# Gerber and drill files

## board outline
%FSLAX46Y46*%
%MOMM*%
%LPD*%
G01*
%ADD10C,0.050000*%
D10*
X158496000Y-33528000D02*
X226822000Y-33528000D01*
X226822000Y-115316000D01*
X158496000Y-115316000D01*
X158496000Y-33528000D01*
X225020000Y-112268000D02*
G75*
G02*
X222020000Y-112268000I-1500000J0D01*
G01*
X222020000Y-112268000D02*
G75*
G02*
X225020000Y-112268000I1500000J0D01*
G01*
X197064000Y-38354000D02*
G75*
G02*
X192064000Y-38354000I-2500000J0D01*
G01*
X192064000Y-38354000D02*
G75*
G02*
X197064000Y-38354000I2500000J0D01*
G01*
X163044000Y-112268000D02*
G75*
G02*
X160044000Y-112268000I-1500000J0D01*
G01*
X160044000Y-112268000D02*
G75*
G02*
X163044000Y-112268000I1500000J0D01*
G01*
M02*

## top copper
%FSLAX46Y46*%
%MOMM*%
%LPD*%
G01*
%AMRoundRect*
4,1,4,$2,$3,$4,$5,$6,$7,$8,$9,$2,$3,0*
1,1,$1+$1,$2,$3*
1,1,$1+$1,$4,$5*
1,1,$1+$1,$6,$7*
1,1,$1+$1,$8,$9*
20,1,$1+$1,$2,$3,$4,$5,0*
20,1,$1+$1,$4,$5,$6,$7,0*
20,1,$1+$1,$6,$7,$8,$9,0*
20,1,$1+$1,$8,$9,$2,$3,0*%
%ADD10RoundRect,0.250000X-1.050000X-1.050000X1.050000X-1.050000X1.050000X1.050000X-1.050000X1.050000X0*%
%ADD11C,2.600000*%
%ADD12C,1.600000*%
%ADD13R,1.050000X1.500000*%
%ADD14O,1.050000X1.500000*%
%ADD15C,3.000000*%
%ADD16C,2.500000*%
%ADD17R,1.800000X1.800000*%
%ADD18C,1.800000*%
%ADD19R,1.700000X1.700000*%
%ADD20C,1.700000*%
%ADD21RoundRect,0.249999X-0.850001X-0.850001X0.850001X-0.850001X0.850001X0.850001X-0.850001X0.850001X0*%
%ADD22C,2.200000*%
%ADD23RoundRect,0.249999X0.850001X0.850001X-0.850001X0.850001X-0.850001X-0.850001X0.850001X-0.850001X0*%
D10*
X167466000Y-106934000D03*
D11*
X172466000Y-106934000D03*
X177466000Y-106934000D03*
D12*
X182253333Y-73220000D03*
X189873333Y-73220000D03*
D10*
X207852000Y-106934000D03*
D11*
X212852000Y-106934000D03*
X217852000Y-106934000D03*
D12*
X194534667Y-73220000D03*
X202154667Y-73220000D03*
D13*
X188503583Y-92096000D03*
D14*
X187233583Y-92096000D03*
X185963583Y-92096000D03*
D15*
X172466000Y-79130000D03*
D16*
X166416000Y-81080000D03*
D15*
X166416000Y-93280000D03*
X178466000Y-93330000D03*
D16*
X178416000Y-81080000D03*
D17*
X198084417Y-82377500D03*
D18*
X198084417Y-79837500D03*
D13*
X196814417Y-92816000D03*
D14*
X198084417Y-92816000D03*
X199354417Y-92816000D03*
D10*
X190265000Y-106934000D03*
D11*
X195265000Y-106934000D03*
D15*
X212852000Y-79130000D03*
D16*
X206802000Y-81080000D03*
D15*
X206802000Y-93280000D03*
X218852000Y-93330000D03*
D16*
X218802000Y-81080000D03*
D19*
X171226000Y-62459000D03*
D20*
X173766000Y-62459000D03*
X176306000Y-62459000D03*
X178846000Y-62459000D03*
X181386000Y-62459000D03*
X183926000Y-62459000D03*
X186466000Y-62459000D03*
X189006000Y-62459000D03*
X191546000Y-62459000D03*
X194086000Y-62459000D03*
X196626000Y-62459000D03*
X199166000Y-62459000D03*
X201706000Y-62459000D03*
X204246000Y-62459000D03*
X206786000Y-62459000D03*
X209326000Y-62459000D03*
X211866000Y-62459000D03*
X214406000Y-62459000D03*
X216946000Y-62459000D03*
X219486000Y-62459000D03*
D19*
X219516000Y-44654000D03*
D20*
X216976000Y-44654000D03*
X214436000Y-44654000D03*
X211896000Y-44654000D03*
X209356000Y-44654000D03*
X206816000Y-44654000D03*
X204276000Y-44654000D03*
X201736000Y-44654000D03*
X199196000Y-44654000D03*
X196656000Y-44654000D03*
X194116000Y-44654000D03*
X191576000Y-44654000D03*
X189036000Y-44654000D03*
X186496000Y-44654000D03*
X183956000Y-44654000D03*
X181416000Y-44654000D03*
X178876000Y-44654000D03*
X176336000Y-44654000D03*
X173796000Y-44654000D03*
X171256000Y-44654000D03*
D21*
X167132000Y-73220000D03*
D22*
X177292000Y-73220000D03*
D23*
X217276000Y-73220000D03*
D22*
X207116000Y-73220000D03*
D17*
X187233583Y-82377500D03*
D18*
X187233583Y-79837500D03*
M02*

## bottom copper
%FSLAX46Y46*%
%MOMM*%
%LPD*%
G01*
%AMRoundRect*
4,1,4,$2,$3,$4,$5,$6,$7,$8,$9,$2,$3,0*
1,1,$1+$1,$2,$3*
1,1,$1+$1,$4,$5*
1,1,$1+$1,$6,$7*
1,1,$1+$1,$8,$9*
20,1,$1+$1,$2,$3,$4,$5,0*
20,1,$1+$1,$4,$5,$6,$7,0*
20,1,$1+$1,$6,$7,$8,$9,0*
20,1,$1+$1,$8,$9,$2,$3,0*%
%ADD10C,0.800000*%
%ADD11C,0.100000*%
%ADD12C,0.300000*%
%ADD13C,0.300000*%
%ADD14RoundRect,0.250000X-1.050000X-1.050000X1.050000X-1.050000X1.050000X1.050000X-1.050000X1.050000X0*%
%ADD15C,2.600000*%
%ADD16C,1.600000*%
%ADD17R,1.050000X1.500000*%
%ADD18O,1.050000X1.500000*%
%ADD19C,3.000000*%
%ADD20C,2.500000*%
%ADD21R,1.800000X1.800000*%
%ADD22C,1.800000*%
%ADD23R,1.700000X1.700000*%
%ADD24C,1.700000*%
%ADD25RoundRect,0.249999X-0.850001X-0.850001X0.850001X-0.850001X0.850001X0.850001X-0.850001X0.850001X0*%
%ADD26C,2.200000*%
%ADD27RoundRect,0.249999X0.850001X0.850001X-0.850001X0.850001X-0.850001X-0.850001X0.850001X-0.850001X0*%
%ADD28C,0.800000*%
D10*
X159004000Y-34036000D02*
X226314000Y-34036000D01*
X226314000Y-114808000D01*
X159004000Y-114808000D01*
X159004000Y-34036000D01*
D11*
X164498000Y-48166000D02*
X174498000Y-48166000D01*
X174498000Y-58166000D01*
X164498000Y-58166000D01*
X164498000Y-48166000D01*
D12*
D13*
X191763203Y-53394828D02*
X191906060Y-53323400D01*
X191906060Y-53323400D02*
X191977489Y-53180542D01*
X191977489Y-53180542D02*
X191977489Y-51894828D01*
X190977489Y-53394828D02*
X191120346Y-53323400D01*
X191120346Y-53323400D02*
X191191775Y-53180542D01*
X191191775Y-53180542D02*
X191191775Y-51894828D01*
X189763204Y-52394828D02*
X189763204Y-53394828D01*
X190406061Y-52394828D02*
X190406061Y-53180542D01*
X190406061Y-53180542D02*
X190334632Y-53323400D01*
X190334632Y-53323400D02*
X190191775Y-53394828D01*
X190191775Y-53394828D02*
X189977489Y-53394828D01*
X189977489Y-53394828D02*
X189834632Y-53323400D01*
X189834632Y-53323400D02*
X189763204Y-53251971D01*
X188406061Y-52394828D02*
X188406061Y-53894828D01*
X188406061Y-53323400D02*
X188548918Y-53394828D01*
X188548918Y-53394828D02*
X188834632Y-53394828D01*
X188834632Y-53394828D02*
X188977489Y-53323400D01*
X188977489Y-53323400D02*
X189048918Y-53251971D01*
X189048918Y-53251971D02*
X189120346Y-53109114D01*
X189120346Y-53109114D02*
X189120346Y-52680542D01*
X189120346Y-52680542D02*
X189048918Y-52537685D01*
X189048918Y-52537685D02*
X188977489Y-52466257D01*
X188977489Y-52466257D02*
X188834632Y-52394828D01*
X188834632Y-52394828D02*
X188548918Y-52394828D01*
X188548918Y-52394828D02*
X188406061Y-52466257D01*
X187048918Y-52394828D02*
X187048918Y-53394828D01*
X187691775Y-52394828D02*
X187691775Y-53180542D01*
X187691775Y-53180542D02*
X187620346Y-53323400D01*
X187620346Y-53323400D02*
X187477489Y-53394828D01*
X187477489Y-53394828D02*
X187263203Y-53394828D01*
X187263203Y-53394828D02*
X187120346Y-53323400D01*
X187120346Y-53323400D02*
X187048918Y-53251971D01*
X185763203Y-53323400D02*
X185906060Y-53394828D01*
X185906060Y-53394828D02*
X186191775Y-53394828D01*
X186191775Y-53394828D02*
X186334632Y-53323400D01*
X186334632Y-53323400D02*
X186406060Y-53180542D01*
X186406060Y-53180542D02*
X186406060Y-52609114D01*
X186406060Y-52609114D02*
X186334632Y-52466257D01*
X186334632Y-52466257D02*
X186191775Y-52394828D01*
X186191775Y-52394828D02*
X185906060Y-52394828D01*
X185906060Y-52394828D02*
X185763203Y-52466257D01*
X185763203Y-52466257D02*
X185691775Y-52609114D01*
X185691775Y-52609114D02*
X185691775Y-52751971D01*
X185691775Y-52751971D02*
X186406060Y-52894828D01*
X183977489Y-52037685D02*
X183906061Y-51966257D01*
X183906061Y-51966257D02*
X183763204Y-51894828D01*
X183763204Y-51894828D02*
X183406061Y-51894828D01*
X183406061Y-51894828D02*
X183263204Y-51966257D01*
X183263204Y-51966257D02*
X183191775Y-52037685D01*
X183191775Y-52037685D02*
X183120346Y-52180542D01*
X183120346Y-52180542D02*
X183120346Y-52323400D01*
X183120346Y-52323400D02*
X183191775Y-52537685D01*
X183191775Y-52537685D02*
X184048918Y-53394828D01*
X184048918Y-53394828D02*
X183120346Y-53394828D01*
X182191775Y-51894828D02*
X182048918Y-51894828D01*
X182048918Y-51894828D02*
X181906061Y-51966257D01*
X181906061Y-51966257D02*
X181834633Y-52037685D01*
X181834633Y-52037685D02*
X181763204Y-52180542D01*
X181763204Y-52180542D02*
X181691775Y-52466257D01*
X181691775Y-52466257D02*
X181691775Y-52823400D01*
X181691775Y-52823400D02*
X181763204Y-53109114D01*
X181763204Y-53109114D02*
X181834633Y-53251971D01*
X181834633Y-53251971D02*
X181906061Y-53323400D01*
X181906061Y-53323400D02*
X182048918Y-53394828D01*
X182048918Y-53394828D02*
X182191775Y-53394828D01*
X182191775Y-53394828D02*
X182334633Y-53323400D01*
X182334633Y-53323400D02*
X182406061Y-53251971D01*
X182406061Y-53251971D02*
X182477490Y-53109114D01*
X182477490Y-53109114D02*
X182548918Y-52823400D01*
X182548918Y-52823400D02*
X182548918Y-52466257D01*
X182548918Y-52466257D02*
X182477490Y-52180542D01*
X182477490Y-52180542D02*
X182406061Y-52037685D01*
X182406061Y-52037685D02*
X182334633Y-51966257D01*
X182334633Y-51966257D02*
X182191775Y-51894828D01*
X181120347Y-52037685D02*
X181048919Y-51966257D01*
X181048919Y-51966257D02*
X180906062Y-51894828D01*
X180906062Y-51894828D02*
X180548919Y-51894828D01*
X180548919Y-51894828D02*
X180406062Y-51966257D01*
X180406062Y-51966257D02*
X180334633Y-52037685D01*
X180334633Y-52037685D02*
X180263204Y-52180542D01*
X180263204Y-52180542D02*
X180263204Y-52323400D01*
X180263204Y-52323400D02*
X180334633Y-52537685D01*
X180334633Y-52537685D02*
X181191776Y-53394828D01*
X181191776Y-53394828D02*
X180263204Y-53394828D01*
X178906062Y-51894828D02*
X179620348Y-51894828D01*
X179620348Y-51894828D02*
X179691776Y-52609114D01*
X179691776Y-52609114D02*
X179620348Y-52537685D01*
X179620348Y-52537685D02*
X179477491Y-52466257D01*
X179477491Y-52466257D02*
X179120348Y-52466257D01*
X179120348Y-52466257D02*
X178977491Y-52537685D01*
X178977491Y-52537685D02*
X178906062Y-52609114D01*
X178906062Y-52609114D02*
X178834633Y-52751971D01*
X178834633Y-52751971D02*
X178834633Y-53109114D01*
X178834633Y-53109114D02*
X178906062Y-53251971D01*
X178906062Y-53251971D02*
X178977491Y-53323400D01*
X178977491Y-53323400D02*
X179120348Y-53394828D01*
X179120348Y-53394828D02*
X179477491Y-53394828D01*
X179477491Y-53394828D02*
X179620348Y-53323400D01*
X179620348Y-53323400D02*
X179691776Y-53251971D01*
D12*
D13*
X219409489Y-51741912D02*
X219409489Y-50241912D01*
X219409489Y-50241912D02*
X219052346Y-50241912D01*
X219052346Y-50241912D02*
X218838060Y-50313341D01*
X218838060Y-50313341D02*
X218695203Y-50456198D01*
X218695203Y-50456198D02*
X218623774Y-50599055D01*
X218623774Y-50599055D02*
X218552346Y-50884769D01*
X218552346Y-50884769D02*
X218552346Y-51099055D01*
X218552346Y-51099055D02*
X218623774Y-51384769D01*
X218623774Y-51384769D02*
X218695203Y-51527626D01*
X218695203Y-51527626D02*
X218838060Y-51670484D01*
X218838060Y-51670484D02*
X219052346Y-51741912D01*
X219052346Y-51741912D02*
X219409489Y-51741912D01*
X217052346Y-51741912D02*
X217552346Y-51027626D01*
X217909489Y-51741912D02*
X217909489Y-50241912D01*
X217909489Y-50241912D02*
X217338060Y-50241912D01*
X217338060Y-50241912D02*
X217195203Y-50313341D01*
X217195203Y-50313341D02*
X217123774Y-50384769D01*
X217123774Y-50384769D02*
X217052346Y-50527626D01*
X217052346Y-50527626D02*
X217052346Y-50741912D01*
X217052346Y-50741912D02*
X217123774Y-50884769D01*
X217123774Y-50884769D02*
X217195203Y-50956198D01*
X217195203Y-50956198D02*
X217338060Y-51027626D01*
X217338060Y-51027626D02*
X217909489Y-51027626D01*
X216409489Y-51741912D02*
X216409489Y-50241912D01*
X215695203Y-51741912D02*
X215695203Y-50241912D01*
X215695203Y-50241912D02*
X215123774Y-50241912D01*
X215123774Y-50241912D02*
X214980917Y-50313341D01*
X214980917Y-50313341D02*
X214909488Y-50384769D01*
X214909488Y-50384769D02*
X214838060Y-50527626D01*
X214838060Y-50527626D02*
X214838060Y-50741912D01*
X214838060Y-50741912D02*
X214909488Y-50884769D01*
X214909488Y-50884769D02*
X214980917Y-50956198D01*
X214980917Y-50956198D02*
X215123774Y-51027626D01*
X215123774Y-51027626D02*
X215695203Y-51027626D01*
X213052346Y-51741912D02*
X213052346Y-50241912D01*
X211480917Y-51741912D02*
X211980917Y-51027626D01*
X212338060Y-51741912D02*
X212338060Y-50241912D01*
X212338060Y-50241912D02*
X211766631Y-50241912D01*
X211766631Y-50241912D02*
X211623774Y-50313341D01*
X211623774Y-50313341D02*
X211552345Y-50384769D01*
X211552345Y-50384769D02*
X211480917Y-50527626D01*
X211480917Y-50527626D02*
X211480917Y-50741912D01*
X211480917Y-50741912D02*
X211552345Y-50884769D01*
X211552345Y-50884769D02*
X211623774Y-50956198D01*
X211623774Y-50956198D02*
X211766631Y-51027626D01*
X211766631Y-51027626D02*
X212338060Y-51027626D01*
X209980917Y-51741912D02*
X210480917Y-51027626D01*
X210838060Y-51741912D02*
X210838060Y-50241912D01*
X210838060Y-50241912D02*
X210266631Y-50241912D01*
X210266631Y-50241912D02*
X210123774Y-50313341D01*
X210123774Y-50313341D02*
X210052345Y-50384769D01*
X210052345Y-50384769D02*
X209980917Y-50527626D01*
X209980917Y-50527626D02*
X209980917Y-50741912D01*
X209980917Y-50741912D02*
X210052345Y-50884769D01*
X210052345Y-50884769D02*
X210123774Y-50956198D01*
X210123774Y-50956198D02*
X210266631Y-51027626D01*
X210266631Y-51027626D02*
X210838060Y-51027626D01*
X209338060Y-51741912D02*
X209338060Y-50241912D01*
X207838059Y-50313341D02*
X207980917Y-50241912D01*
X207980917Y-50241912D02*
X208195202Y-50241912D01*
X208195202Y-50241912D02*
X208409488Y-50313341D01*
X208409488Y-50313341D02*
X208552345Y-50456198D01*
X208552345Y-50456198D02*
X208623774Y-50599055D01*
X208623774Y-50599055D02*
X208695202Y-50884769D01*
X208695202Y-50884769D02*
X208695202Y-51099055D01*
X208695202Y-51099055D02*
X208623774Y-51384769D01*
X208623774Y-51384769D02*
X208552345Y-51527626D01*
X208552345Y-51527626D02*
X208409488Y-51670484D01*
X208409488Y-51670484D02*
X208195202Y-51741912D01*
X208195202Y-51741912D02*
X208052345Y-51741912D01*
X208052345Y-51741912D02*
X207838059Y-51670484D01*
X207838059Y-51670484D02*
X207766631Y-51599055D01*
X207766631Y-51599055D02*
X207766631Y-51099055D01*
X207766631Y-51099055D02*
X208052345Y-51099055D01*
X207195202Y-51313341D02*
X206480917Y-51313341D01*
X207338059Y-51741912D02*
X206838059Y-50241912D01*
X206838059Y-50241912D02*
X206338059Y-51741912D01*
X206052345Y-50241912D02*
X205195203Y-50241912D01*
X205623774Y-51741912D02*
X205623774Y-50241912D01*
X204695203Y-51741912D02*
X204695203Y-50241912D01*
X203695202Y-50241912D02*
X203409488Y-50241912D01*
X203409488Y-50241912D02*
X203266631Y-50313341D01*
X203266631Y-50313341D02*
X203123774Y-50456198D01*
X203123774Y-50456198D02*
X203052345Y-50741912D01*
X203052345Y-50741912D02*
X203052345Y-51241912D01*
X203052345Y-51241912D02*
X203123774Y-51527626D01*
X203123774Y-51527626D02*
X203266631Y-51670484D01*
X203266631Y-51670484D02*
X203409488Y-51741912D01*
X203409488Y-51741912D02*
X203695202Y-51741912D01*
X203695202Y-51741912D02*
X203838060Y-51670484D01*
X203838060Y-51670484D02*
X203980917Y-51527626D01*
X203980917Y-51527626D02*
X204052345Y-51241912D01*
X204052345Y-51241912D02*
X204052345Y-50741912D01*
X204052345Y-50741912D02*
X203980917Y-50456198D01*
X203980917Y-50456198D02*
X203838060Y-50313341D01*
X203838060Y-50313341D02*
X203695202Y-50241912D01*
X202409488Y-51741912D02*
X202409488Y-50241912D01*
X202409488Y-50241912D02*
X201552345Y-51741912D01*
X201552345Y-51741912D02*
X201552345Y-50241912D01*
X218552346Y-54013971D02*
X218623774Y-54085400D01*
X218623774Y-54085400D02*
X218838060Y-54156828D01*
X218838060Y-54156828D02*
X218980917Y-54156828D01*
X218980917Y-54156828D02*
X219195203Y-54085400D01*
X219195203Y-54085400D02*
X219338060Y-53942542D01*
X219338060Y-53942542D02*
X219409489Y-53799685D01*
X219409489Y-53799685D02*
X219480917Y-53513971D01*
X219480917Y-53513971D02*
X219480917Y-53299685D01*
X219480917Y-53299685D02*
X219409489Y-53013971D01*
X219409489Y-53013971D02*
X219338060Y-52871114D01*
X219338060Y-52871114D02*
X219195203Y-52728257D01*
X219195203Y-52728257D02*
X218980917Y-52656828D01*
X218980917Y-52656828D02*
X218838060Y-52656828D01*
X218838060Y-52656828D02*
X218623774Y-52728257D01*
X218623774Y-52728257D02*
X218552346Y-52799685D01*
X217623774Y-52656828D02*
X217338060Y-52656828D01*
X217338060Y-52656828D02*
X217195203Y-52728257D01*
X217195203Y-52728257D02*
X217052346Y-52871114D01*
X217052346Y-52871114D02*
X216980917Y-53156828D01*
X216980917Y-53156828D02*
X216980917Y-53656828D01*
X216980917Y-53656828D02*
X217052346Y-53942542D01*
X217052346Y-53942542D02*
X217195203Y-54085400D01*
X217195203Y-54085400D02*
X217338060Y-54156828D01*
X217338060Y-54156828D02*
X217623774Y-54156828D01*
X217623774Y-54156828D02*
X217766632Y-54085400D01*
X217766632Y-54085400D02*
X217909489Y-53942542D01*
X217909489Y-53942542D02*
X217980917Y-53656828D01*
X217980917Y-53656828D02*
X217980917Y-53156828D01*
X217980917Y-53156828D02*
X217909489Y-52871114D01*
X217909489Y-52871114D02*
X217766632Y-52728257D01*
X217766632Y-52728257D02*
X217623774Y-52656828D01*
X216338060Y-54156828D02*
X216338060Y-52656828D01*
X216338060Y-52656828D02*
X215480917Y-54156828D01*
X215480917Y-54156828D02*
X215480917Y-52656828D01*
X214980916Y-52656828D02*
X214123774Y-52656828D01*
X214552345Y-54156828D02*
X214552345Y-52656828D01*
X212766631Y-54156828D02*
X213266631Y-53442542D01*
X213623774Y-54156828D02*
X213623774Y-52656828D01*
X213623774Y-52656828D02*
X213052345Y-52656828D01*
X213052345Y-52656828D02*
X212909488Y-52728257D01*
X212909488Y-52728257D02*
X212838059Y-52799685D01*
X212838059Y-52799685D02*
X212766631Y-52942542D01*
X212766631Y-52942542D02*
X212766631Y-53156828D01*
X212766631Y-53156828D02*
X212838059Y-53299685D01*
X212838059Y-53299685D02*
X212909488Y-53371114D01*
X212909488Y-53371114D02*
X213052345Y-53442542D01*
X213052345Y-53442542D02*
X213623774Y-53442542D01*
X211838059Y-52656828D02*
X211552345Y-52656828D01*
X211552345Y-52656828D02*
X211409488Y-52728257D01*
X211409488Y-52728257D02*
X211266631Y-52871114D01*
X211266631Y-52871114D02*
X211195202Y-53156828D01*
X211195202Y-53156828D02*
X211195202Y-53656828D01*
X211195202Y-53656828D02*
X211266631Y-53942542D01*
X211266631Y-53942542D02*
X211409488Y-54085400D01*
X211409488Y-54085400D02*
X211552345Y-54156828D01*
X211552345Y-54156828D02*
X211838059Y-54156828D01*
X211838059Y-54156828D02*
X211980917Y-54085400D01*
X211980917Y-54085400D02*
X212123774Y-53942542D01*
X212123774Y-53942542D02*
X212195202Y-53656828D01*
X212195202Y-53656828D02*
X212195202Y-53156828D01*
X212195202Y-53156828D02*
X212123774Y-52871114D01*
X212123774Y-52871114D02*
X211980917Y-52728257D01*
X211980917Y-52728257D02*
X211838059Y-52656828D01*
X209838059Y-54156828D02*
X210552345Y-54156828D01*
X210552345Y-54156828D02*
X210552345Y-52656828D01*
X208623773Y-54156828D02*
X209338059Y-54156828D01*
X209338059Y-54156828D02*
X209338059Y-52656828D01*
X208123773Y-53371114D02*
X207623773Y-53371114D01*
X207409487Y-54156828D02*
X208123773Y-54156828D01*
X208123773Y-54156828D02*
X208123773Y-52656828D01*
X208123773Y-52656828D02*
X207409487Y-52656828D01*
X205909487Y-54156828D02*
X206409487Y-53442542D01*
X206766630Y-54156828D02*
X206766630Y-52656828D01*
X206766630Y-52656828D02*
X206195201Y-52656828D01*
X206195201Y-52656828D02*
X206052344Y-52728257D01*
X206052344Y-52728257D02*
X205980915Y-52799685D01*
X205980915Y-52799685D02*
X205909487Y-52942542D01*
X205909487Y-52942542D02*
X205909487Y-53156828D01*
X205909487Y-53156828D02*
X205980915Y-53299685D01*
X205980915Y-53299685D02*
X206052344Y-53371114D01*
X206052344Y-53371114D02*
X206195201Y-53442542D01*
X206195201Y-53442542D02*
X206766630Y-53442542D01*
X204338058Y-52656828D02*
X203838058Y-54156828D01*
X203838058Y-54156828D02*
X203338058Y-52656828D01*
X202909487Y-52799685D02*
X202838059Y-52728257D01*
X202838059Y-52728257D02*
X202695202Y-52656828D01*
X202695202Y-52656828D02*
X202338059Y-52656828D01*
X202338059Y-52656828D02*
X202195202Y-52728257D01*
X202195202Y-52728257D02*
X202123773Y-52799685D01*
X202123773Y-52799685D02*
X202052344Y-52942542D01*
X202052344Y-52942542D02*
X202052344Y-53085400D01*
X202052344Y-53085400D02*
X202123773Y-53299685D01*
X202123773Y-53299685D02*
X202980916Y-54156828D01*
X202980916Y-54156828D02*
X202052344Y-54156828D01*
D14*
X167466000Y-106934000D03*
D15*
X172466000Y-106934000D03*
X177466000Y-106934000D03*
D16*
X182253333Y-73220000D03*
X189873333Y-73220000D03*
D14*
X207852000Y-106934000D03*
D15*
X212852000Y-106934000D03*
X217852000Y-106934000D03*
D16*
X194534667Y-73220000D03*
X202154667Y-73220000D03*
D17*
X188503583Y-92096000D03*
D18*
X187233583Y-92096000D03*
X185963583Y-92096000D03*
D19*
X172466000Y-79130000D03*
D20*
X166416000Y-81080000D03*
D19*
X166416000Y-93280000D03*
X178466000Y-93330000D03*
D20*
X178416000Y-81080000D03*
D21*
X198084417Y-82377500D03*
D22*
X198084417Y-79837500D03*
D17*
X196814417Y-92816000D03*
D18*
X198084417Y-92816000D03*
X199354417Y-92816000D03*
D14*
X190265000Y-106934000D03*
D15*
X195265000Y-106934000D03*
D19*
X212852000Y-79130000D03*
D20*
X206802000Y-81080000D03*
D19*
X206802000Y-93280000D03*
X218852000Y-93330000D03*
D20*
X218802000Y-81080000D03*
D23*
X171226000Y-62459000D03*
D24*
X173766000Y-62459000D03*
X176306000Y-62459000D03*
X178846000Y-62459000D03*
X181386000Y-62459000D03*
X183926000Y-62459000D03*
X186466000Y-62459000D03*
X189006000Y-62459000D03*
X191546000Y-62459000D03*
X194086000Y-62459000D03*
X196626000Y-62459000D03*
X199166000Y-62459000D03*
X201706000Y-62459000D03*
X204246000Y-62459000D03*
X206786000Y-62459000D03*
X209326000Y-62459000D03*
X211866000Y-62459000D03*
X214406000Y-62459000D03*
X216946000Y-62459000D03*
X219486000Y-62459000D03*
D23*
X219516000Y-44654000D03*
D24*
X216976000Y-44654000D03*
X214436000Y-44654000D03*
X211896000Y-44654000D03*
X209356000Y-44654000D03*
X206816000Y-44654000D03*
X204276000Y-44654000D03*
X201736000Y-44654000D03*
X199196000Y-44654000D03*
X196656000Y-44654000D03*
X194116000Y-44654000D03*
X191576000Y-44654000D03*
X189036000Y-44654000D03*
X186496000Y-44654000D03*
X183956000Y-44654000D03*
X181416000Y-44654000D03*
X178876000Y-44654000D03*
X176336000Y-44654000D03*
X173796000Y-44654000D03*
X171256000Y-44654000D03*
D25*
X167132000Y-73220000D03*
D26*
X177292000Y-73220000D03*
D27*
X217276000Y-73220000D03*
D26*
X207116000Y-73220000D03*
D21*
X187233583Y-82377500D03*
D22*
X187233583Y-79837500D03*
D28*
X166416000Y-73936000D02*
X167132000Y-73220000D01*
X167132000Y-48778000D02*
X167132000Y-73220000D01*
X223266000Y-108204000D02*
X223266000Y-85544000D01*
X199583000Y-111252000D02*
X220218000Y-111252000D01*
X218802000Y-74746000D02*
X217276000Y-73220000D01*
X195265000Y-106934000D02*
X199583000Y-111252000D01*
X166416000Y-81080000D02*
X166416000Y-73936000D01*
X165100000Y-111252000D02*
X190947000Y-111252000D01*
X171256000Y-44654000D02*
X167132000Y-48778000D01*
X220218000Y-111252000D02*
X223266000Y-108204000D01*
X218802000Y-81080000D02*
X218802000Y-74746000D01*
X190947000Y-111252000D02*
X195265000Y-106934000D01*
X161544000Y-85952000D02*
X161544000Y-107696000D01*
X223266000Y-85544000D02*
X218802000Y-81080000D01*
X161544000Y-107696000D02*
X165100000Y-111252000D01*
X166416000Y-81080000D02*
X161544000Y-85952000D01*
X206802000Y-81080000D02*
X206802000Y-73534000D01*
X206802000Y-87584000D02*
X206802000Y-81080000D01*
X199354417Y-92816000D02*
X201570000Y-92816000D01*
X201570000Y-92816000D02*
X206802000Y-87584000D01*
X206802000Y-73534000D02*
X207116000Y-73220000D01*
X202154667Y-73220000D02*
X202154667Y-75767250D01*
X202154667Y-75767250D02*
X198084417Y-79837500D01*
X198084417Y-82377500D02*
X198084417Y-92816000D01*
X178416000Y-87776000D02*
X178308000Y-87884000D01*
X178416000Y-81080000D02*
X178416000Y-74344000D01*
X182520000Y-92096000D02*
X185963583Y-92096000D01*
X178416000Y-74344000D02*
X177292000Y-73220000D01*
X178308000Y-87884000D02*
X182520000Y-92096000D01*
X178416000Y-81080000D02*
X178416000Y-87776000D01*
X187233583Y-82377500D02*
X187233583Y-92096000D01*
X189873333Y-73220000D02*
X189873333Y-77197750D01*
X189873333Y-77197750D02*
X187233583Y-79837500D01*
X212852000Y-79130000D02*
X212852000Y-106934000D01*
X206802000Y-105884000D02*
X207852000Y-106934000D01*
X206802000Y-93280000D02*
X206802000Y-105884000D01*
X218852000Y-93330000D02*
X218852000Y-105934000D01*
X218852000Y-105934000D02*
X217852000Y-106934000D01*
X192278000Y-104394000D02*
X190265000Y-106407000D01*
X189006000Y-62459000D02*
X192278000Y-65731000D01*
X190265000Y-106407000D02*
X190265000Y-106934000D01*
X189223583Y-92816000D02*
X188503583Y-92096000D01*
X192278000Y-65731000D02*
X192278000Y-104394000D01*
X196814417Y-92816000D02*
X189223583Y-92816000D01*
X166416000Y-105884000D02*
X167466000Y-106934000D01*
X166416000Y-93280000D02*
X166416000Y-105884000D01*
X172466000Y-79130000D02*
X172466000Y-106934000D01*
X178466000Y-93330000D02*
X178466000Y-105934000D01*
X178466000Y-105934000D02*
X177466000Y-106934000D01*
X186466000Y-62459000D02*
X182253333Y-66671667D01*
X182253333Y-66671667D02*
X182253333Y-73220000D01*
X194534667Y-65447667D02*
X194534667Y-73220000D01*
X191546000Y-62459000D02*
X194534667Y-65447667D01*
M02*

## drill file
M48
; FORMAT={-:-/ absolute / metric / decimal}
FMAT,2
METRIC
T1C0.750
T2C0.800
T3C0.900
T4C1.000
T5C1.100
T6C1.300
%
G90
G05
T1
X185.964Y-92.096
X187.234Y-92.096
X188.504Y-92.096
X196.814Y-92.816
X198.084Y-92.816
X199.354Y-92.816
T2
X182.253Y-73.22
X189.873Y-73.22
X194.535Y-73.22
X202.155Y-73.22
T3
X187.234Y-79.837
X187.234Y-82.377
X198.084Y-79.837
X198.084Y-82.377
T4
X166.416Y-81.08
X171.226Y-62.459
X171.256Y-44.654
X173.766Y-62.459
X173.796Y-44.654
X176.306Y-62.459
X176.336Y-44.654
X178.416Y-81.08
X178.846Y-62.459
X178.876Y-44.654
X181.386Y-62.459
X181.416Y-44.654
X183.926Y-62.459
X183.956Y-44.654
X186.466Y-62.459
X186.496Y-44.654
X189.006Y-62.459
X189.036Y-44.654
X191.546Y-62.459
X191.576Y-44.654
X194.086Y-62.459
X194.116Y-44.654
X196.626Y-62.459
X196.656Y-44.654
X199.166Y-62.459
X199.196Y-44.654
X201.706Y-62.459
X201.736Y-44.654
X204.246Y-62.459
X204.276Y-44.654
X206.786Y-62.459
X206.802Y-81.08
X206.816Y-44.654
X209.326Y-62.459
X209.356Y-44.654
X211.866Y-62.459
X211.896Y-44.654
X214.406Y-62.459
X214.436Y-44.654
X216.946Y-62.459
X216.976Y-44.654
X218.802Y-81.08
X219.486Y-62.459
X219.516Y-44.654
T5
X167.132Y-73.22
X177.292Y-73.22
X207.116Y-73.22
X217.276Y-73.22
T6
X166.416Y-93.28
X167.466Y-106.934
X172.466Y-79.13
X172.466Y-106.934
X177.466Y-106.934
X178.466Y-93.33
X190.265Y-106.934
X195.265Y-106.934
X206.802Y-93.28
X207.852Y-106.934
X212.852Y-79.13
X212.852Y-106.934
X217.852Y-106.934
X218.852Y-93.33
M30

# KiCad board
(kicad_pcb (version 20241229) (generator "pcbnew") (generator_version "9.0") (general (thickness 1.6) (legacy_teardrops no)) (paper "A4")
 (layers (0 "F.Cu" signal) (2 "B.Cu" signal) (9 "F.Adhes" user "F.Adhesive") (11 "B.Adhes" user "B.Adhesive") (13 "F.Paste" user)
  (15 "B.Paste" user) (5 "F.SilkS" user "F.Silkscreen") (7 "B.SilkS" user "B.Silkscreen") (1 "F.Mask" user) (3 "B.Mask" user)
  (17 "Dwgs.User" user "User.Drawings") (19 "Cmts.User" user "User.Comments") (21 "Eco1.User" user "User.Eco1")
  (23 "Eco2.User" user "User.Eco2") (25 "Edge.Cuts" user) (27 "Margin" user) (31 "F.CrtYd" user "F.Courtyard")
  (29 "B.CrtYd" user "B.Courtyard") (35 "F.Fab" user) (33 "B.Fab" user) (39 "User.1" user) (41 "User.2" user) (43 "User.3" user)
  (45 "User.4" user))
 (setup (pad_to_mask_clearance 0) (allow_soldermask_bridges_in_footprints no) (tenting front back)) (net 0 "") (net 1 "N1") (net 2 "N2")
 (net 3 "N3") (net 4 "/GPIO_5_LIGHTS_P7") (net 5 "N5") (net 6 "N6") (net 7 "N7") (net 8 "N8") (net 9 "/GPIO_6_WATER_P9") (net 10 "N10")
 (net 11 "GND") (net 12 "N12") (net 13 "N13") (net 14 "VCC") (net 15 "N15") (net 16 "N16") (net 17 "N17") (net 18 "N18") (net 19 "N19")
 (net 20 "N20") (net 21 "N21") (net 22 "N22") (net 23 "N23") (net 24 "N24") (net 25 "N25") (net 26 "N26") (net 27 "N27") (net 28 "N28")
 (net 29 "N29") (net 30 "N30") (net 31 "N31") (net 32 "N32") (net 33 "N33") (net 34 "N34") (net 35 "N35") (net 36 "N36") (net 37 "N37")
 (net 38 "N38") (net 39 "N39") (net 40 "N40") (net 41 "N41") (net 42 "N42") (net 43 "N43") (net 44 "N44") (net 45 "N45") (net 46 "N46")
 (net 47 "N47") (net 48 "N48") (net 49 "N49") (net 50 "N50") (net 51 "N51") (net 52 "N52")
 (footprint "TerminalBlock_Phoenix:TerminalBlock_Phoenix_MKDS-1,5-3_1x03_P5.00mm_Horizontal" (layer "F.Cu") (at 167.466 106.934)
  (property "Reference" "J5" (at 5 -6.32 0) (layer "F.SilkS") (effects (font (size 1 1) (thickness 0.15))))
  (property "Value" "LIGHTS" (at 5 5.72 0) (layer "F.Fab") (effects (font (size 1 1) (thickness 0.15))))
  (pad "1" thru_hole roundrect (at 0 0) (size 2.6 2.6) (drill 1.3) (layers "*.Cu" "*.Mask") (remove_unused_layers no)
   (roundrect_rratio 0.096154) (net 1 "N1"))
  (pad "2" thru_hole circle (at 5 0) (size 2.6 2.6) (drill 1.3) (layers "*.Cu" "*.Mask") (remove_unused_layers no) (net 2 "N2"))
  (pad "3" thru_hole circle (at 10 0) (size 2.6 2.6) (drill 1.3) (layers "*.Cu" "*.Mask") (remove_unused_layers no) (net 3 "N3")))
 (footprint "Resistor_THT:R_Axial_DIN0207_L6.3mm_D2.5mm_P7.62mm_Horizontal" (layer "F.Cu") (at 182.253333 73.22)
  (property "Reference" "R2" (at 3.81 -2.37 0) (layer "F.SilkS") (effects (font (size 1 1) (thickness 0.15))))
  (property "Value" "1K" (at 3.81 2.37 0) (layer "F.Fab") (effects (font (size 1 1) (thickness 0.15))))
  (pad "1" thru_hole circle (at 0 0) (size 1.6 1.6) (drill 0.8) (layers "*.Cu" "*.Mask") (remove_unused_layers no)
   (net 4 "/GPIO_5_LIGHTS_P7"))
  (pad "2" thru_hole circle (at 7.62 0) (size 1.6 1.6) (drill 0.8) (layers "*.Cu" "*.Mask") (remove_unused_layers no) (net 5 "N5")))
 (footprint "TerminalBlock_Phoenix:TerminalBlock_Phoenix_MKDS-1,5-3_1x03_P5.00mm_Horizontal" (layer "F.Cu") (at 207.852 106.934)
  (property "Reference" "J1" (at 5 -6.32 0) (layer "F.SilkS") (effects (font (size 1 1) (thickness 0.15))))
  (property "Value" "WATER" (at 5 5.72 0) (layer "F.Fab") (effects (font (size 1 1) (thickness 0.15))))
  (pad "1" thru_hole roundrect (at 0 0) (size 2.6 2.6) (drill 1.3) (layers "*.Cu" "*.Mask") (remove_unused_layers no)
   (roundrect_rratio 0.096154) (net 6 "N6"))
  (pad "2" thru_hole circle (at 5 0) (size 2.6 2.6) (drill 1.3) (layers "*.Cu" "*.Mask") (remove_unused_layers no) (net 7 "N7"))
  (pad "3" thru_hole circle (at 10 0) (size 2.6 2.6) (drill 1.3) (layers "*.Cu" "*.Mask") (remove_unused_layers no) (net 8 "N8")))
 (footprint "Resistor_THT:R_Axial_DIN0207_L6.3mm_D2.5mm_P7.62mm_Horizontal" (layer "F.Cu") (at 194.534667 73.22)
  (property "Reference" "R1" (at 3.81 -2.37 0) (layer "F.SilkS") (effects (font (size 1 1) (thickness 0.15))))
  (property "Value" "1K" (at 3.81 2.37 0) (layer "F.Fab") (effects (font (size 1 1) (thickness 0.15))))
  (pad "1" thru_hole circle (at 0 0) (size 1.6 1.6) (drill 0.8) (layers "*.Cu" "*.Mask") (remove_unused_layers no)
   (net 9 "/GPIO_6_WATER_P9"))
  (pad "2" thru_hole circle (at 7.62 0) (size 1.6 1.6) (drill 0.8) (layers "*.Cu" "*.Mask") (remove_unused_layers no) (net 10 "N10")))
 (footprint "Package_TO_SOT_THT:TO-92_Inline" (layer "F.Cu") (at 188.503583 92.096 180)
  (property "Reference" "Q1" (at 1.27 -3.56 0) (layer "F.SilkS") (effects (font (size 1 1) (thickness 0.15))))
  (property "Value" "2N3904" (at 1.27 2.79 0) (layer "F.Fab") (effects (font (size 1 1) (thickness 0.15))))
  (pad "1" thru_hole rect (at 0 0 180) (size 1.05 1.5) (drill 0.75) (layers "*.Cu" "*.Mask") (remove_unused_layers no) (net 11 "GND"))
  (pad "2" thru_hole oval (at 1.27 0 180) (size 1.05 1.5) (drill 0.75) (layers "*.Cu" "*.Mask") (remove_unused_layers no) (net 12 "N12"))
  (pad "3" thru_hole oval (at 2.54 0 180) (size 1.05 1.5) (drill 0.75) (layers "*.Cu" "*.Mask") (remove_unused_layers no) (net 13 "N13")))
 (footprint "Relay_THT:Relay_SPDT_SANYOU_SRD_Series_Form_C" (layer "F.Cu") (at 172.466 79.13 -90)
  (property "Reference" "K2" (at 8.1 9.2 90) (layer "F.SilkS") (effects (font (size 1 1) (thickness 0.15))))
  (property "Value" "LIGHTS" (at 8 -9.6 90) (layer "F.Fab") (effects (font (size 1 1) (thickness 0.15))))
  (pad "1" thru_hole circle (at 0 0) (size 3 3) (drill 1.3) (layers "*.Cu" "*.Mask") (remove_unused_layers no) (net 2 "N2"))
  (pad "2" thru_hole circle (at 1.95 6.05) (size 2.5 2.5) (drill 1) (layers "*.Cu" "*.Mask") (remove_unused_layers no) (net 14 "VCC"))
  (pad "3" thru_hole circle (at 14.15 6.05) (size 3 3) (drill 1.3) (layers "*.Cu" "*.Mask") (remove_unused_layers no) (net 1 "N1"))
  (pad "4" thru_hole circle (at 14.2 -6) (size 3 3) (drill 1.3) (layers "*.Cu" "*.Mask") (remove_unused_layers no) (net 3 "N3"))
  (pad "5" thru_hole circle (at 1.95 -5.95) (size 2.5 2.5) (drill 1) (layers "*.Cu" "*.Mask") (remove_unused_layers no) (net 13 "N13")))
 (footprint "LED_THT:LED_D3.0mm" (layer "F.Cu") (at 198.084417 82.3775 90)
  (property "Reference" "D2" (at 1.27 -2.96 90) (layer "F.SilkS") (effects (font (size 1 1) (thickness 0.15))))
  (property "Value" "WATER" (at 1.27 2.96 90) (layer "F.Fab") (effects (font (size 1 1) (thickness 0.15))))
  (pad "1" thru_hole rect (at 0 0 90) (size 1.8 1.8) (drill 0.9) (layers "*.Cu" "*.Mask") (remove_unused_layers no) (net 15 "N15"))
  (pad "2" thru_hole circle (at 2.54 0 90) (size 1.8 1.8) (drill 0.9) (layers "*.Cu" "*.Mask") (remove_unused_layers no) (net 10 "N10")))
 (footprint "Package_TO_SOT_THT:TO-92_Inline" (layer "F.Cu") (at 196.814417 92.816)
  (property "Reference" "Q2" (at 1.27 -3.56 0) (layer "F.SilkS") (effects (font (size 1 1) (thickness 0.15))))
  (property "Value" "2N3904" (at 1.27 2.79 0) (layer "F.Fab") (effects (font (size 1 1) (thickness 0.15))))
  (pad "1" thru_hole rect (at 0 0) (size 1.05 1.5) (drill 0.75) (layers "*.Cu" "*.Mask") (remove_unused_layers no) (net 11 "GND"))
  (pad "2" thru_hole oval (at 1.27 0) (size 1.05 1.5) (drill 0.75) (layers "*.Cu" "*.Mask") (remove_unused_layers no) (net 15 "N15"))
  (pad "3" thru_hole oval (at 2.54 0) (size 1.05 1.5) (drill 0.75) (layers "*.Cu" "*.Mask") (remove_unused_layers no) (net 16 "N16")))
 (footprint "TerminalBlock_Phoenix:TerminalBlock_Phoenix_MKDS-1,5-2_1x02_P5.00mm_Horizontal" (layer "F.Cu") (at 190.265 106.934)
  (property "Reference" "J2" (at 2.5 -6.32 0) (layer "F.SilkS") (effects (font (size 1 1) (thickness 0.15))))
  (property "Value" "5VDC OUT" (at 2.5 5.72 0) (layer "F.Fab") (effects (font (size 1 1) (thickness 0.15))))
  (pad "1" thru_hole roundrect (at 0 0) (size 2.6 2.6) (drill 1.3) (layers "*.Cu" "*.Mask") (remove_unused_layers no)
   (roundrect_rratio 0.096154) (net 11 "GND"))
  (pad "2" thru_hole circle (at 5 0) (size 2.6 2.6) (drill 1.3) (layers "*.Cu" "*.Mask") (remove_unused_layers no) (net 14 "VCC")))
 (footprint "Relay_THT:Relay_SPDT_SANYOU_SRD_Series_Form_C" (layer "F.Cu") (at 212.852 79.13 -90)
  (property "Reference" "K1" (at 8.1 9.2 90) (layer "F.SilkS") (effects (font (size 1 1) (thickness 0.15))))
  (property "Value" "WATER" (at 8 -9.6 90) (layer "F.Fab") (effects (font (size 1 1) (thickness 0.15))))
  (pad "1" thru_hole circle (at 0 0) (size 3 3) (drill 1.3) (layers "*.Cu" "*.Mask") (remove_unused_layers no) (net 7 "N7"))
  (pad "2" thru_hole circle (at 1.95 6.05) (size 2.5 2.5) (drill 1) (layers "*.Cu" "*.Mask") (remove_unused_layers no) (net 16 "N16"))
  (pad "3" thru_hole circle (at 14.15 6.05) (size 3 3) (drill 1.3) (layers "*.Cu" "*.Mask") (remove_unused_layers no) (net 6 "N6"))
  (pad "4" thru_hole circle (at 14.2 -6) (size 3 3) (drill 1.3) (layers "*.Cu" "*.Mask") (remove_unused_layers no) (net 8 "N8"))
  (pad "5" thru_hole circle (at 1.95 -5.95) (size 2.5 2.5) (drill 1) (layers "*.Cu" "*.Mask") (remove_unused_layers no) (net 14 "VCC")))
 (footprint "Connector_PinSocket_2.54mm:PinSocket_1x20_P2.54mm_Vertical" (layer "F.Cu") (at 171.226 62.459 90)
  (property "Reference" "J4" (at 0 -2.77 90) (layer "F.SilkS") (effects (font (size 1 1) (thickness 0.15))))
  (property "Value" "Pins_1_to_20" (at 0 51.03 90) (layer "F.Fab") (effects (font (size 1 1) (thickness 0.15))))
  (pad "1" thru_hole rect (at 0 0 90) (size 1.7 1.7) (drill 1) (layers "*.Cu" "*.Mask") (remove_unused_layers no) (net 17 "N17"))
  (pad "2" thru_hole circle (at 0 2.54 90) (size 1.7 1.7) (drill 1) (layers "*.Cu" "*.Mask") (remove_unused_layers no) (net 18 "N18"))
  (pad "3" thru_hole circle (at 0 5.08 90) (size 1.7 1.7) (drill 1) (layers "*.Cu" "*.Mask") (remove_unused_layers no) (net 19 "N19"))
  (pad "4" thru_hole circle (at 0 7.62 90) (size 1.7 1.7) (drill 1) (layers "*.Cu" "*.Mask") (remove_unused_layers no) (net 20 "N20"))
  (pad "5" thru_hole circle (at 0 10.16 90) (size 1.7 1.7) (drill 1) (layers "*.Cu" "*.Mask") (remove_unused_layers no) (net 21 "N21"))
  (pad "6" thru_hole circle (at 0 12.7 90) (size 1.7 1.7) (drill 1) (layers "*.Cu" "*.Mask") (remove_unused_layers no) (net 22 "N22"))
  (pad "7" thru_hole circle (at 0 15.24 90) (size 1.7 1.7) (drill 1) (layers "*.Cu" "*.Mask") (remove_unused_layers no)
   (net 4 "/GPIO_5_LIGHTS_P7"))
  (pad "8" thru_hole circle (at 0 17.78 90) (size 1.7 1.7) (drill 1) (layers "*.Cu" "*.Mask") (remove_unused_layers no) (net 11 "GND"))
  (pad "9" thru_hole circle (at 0 20.32 90) (size 1.7 1.7) (drill 1) (layers "*.Cu" "*.Mask") (remove_unused_layers no)
   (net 9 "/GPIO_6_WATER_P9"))
  (pad "10" thru_hole circle (at 0 22.86 90) (size 1.7 1.7) (drill 1) (layers "*.Cu" "*.Mask") (remove_unused_layers no) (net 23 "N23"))
  (pad "11" thru_hole circle (at 0 25.4 90) (size 1.7 1.7) (drill 1) (layers "*.Cu" "*.Mask") (remove_unused_layers no) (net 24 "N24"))
  (pad "12" thru_hole circle (at 0 27.94 90) (size 1.7 1.7) (drill 1) (layers "*.Cu" "*.Mask") (remove_unused_layers no) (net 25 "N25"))
  (pad "13" thru_hole circle (at 0 30.48 90) (size 1.7 1.7) (drill 1) (layers "*.Cu" "*.Mask") (remove_unused_layers no) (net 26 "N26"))
  (pad "14" thru_hole circle (at 0 33.02 90) (size 1.7 1.7) (drill 1) (layers "*.Cu" "*.Mask") (remove_unused_layers no) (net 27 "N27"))
  (pad "15" thru_hole circle (at 0 35.56 90) (size 1.7 1.7) (drill 1) (layers "*.Cu" "*.Mask") (remove_unused_layers no) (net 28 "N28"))
  (pad "16" thru_hole circle (at 0 38.1 90) (size 1.7 1.7) (drill 1) (layers "*.Cu" "*.Mask") (remove_unused_layers no) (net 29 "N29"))
  (pad "17" thru_hole circle (at 0 40.64 90) (size 1.7 1.7) (drill 1) (layers "*.Cu" "*.Mask") (remove_unused_layers no) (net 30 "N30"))
  (pad "18" thru_hole circle (at 0 43.18 90) (size 1.7 1.7) (drill 1) (layers "*.Cu" "*.Mask") (remove_unused_layers no) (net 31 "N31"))
  (pad "19" thru_hole circle (at 0 45.72 90) (size 1.7 1.7) (drill 1) (layers "*.Cu" "*.Mask") (remove_unused_layers no) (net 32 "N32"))
  (pad "20" thru_hole circle (at 0 48.26 90) (size 1.7 1.7) (drill 1) (layers "*.Cu" "*.Mask") (remove_unused_layers no) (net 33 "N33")))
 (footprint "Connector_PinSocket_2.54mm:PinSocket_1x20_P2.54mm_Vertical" (layer "F.Cu") (at 219.516 44.654 -90)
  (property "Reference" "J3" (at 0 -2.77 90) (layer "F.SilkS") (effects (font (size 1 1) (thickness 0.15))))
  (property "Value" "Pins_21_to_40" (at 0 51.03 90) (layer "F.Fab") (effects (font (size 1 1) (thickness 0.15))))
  (pad "1" thru_hole rect (at 0 0 270) (size 1.7 1.7) (drill 1) (layers "*.Cu" "*.Mask") (remove_unused_layers no) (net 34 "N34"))
  (pad "2" thru_hole circle (at 0 2.54 270) (size 1.7 1.7) (drill 1) (layers "*.Cu" "*.Mask") (remove_unused_layers no) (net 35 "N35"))
  (pad "3" thru_hole circle (at 0 5.08 270) (size 1.7 1.7) (drill 1) (layers "*.Cu" "*.Mask") (remove_unused_layers no) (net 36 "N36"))
  (pad "4" thru_hole circle (at 0 7.62 270) (size 1.7 1.7) (drill 1) (layers "*.Cu" "*.Mask") (remove_unused_layers no) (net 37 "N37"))
  (pad "5" thru_hole circle (at 0 10.16 270) (size 1.7 1.7) (drill 1) (layers "*.Cu" "*.Mask") (remove_unused_layers no) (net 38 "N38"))
  (pad "6" thru_hole circle (at 0 12.7 270) (size 1.7 1.7) (drill 1) (layers "*.Cu" "*.Mask") (remove_unused_layers no) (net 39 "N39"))
  (pad "7" thru_hole circle (at 0 15.24 270) (size 1.7 1.7) (drill 1) (layers "*.Cu" "*.Mask") (remove_unused_layers no) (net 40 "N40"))
  (pad "8" thru_hole circle (at 0 17.78 270) (size 1.7 1.7) (drill 1) (layers "*.Cu" "*.Mask") (remove_unused_layers no) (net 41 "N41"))
  (pad "9" thru_hole circle (at 0 20.32 270) (size 1.7 1.7) (drill 1) (layers "*.Cu" "*.Mask") (remove_unused_layers no) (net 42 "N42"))
  (pad "10" thru_hole circle (at 0 22.86 270) (size 1.7 1.7) (drill 1) (layers "*.Cu" "*.Mask") (remove_unused_layers no) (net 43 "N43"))
  (pad "11" thru_hole circle (at 0 25.4 270) (size 1.7 1.7) (drill 1) (layers "*.Cu" "*.Mask") (remove_unused_layers no) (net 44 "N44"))
  (pad "12" thru_hole circle (at 0 27.94 270) (size 1.7 1.7) (drill 1) (layers "*.Cu" "*.Mask") (remove_unused_layers no) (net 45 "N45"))
  (pad "13" thru_hole circle (at 0 30.48 270) (size 1.7 1.7) (drill 1) (layers "*.Cu" "*.Mask") (remove_unused_layers no) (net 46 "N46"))
  (pad "14" thru_hole circle (at 0 33.02 270) (size 1.7 1.7) (drill 1) (layers "*.Cu" "*.Mask") (remove_unused_layers no) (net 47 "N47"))
  (pad "15" thru_hole circle (at 0 35.56 270) (size 1.7 1.7) (drill 1) (layers "*.Cu" "*.Mask") (remove_unused_layers no) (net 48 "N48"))
  (pad "16" thru_hole circle (at 0 38.1 270) (size 1.7 1.7) (drill 1) (layers "*.Cu" "*.Mask") (remove_unused_layers no) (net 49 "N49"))
  (pad "17" thru_hole circle (at 0 40.64 270) (size 1.7 1.7) (drill 1) (layers "*.Cu" "*.Mask") (remove_unused_layers no) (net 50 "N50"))
  (pad "18" thru_hole circle (at 0 43.18 270) (size 1.7 1.7) (drill 1) (layers "*.Cu" "*.Mask") (remove_unused_layers no) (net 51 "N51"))
  (pad "19" thru_hole circle (at 0 45.72 270) (size 1.7 1.7) (drill 1) (layers "*.Cu" "*.Mask") (remove_unused_layers no) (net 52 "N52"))
  (pad "20" thru_hole circle (at 0 48.26 270) (size 1.7 1.7) (drill 1) (layers "*.Cu" "*.Mask") (remove_unused_layers no) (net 14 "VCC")))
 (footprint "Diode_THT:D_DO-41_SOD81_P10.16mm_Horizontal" (layer "F.Cu") (at 167.132 73.22)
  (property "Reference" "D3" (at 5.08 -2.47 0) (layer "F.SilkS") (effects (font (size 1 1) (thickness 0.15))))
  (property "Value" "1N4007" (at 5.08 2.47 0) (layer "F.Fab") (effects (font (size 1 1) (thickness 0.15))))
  (pad "1" thru_hole roundrect (at 0 0) (size 2.2 2.2) (drill 1.1) (layers "*.Cu" "*.Mask") (remove_unused_layers no)
   (roundrect_rratio 0.113636) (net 14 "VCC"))
  (pad "2" thru_hole circle (at 10.16 0) (size 2.2 2.2) (drill 1.1) (layers "*.Cu" "*.Mask") (remove_unused_layers no) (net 13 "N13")))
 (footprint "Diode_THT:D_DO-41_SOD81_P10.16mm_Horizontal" (layer "F.Cu") (at 217.276 73.22 180)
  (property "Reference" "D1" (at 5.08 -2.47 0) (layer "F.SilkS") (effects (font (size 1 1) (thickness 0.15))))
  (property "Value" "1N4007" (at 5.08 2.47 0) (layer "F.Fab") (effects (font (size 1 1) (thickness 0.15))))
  (pad "1" thru_hole roundrect (at 0 0 180) (size 2.2 2.2) (drill 1.1) (layers "*.Cu" "*.Mask") (remove_unused_layers no)
   (roundrect_rratio 0.113636) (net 14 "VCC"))
  (pad "2" thru_hole circle (at 10.16 0 180) (size 2.2 2.2) (drill 1.1) (layers "*.Cu" "*.Mask") (remove_unused_layers no) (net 16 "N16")))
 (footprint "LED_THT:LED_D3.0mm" (layer "F.Cu") (at 187.233583 82.3775 90)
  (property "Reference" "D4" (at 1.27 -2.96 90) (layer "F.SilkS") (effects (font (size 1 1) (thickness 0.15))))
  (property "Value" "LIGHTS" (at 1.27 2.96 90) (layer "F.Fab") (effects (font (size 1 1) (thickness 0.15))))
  (pad "1" thru_hole rect (at 0 0 90) (size 1.8 1.8) (drill 0.9) (layers "*.Cu" "*.Mask") (remove_unused_layers no) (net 12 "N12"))
  (pad "2" thru_hole circle (at 2.54 0 90) (size 1.8 1.8) (drill 0.9) (layers "*.Cu" "*.Mask") (remove_unused_layers no) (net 5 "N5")))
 (gr_rect (start 159.004 34.036) (end 226.314 114.808) (stroke (width 0.8) (type solid)) (fill no) (layer "B.Cu"))
 (gr_rect (start 164.498 48.166) (end 174.498 58.166) (stroke (width 0.1) (type solid)) (fill no) (layer "B.Cu") (net 14))
 (gr_rect (start 158.496 33.528) (end 226.822 115.316) (stroke (width 0.05) (type default)) (fill no) (layer "Edge.Cuts"))
 (gr_circle (center 223.52 112.268) (end 225.02 112.268) (stroke (width 0.05) (type solid)) (fill no) (layer "Edge.Cuts"))
 (gr_circle (center 194.564 38.354) (end 192.064 38.354) (stroke (width 0.05) (type solid)) (fill no) (layer "Edge.Cuts"))
 (gr_circle (center 161.544 112.268) (end 163.044 112.268) (stroke (width 0.05) (type solid)) (fill no) (layer "Edge.Cuts"))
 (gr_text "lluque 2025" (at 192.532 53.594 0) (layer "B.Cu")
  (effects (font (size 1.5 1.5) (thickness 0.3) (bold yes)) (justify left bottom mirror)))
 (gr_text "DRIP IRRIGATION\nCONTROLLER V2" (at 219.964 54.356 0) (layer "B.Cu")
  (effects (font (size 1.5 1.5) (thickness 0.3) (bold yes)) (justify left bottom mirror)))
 (segment (start 166.416 73.936) (end 167.132 73.22) (width 0.8) (layer "B.Cu") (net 14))
 (segment (start 167.132 48.778) (end 167.132 73.22) (width 0.8) (layer "B.Cu") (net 14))
 (segment (start 223.266 108.204) (end 223.266 85.544) (width 0.8) (layer "B.Cu") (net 14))
 (segment (start 199.583 111.252) (end 220.218 111.252) (width 0.8) (layer "B.Cu") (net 14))
 (segment (start 218.802 74.746) (end 217.276 73.22) (width 0.8) (layer "B.Cu") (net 14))
 (segment (start 195.265 106.934) (end 199.583 111.252) (width 0.8) (layer "B.Cu") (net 14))
 (segment (start 166.416 81.08) (end 166.416 73.936) (width 0.8) (layer "B.Cu") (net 14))
 (segment (start 165.1 111.252) (end 190.947 111.252) (width 0.8) (layer "B.Cu") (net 14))
 (segment (start 171.256 44.654) (end 167.132 48.778) (width 0.8) (layer "B.Cu") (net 14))
 (segment (start 220.218 111.252) (end 223.266 108.204) (width 0.8) (layer "B.Cu") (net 14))
 (segment (start 218.802 81.08) (end 218.802 74.746) (width 0.8) (layer "B.Cu") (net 14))
 (segment (start 190.947 111.252) (end 195.265 106.934) (width 0.8) (layer "B.Cu") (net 14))
 (segment (start 161.544 85.952) (end 161.544 107.696) (width 0.8) (layer "B.Cu") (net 14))
 (segment (start 223.266 85.544) (end 218.802 81.08) (width 0.8) (layer "B.Cu") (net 14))
 (segment (start 161.544 107.696) (end 165.1 111.252) (width 0.8) (layer "B.Cu") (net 14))
 (segment (start 166.416 81.08) (end 161.544 85.952) (width 0.8) (layer "B.Cu") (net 14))
 (segment (start 206.802 81.08) (end 206.802 73.534) (width 0.8) (layer "B.Cu") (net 16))
 (segment (start 206.802 87.584) (end 206.802 81.08) (width 0.8) (layer "B.Cu") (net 16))
 (segment (start 199.354417 92.816) (end 201.57 92.816) (width 0.8) (layer "B.Cu") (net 16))
 (segment (start 201.57 92.816) (end 206.802 87.584) (width 0.8) (layer "B.Cu") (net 16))
 (segment (start 206.802 73.534) (end 207.116 73.22) (width 0.8) (layer "B.Cu") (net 16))
 (segment (start 202.154667 73.22) (end 202.154667 75.76725) (width 0.8) (layer "B.Cu") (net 10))
 (segment (start 202.154667 75.76725) (end 198.084417 79.8375) (width 0.8) (layer "B.Cu") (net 10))
 (segment (start 198.084417 82.3775) (end 198.084417 92.816) (width 0.8) (layer "B.Cu") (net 15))
 (segment (start 178.416 87.776) (end 178.308 87.884) (width 0.8) (layer "B.Cu") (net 13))
 (segment (start 178.416 81.08) (end 178.416 74.344) (width 0.8) (layer "B.Cu") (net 13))
 (segment (start 182.52 92.096) (end 185.963583 92.096) (width 0.8) (layer "B.Cu") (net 13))
 (segment (start 178.416 74.344) (end 177.292 73.22) (width 0.8) (layer "B.Cu") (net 13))
 (segment (start 178.308 87.884) (end 182.52 92.096) (width 0.8) (layer "B.Cu") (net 13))
 (segment (start 178.416 81.08) (end 178.416 87.776) (width 0.8) (layer "B.Cu") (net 13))
 (segment (start 187.233583 82.3775) (end 187.233583 92.096) (width 0.8) (layer "B.Cu") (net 12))
 (segment (start 189.873333 73.22) (end 189.873333 77.19775) (width 0.8) (layer "B.Cu") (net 5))
 (segment (start 189.873333 77.19775) (end 187.233583 79.8375) (width 0.8) (layer "B.Cu") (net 5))
 (segment (start 212.852 79.13) (end 212.852 106.934) (width 0.8) (layer "B.Cu") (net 7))
 (segment (start 206.802 105.884) (end 207.852 106.934) (width 0.8) (layer "B.Cu") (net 6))
 (segment (start 206.802 93.28) (end 206.802 105.884) (width 0.8) (layer "B.Cu") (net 6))
 (segment (start 218.852 93.33) (end 218.852 105.934) (width 0.8) (layer "B.Cu") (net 8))
 (segment (start 218.852 105.934) (end 217.852 106.934) (width 0.8) (layer "B.Cu") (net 8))
 (segment (start 192.278 104.394) (end 190.265 106.407) (width 0.8) (layer "B.Cu") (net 11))
 (segment (start 189.006 62.459) (end 192.278 65.731) (width 0.8) (layer "B.Cu") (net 11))
 (segment (start 190.265 106.407) (end 190.265 106.934) (width 0.8) (layer "B.Cu") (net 11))
 (segment (start 189.223583 92.816) (end 188.503583 92.096) (width 0.8) (layer "B.Cu") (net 11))
 (segment (start 192.278 65.731) (end 192.278 104.394) (width 0.8) (layer "B.Cu") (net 11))
 (segment (start 196.814417 92.816) (end 189.223583 92.816) (width 0.8) (layer "B.Cu") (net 11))
 (segment (start 166.416 105.884) (end 167.466 106.934) (width 0.8) (layer "B.Cu") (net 1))
 (segment (start 166.416 93.28) (end 166.416 105.884) (width 0.8) (layer "B.Cu") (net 1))
 (segment (start 172.466 79.13) (end 172.466 106.934) (width 0.8) (layer "B.Cu") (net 2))
 (segment (start 178.466 93.33) (end 178.466 105.934) (width 0.8) (layer "B.Cu") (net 3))
 (segment (start 178.466 105.934) (end 177.466 106.934) (width 0.8) (layer "B.Cu") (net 3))
 (segment (start 186.466 62.459) (end 182.253333 66.671667) (width 0.8) (layer "B.Cu") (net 4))
 (segment (start 182.253333 66.671667) (end 182.253333 73.22) (width 0.8) (layer "B.Cu") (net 4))
 (segment (start 194.534667 65.447667) (end 194.534667 73.22) (width 0.8) (layer "B.Cu") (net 9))
 (segment (start 191.546 62.459) (end 194.534667 65.447667) (width 0.8) (layer "B.Cu") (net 9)))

